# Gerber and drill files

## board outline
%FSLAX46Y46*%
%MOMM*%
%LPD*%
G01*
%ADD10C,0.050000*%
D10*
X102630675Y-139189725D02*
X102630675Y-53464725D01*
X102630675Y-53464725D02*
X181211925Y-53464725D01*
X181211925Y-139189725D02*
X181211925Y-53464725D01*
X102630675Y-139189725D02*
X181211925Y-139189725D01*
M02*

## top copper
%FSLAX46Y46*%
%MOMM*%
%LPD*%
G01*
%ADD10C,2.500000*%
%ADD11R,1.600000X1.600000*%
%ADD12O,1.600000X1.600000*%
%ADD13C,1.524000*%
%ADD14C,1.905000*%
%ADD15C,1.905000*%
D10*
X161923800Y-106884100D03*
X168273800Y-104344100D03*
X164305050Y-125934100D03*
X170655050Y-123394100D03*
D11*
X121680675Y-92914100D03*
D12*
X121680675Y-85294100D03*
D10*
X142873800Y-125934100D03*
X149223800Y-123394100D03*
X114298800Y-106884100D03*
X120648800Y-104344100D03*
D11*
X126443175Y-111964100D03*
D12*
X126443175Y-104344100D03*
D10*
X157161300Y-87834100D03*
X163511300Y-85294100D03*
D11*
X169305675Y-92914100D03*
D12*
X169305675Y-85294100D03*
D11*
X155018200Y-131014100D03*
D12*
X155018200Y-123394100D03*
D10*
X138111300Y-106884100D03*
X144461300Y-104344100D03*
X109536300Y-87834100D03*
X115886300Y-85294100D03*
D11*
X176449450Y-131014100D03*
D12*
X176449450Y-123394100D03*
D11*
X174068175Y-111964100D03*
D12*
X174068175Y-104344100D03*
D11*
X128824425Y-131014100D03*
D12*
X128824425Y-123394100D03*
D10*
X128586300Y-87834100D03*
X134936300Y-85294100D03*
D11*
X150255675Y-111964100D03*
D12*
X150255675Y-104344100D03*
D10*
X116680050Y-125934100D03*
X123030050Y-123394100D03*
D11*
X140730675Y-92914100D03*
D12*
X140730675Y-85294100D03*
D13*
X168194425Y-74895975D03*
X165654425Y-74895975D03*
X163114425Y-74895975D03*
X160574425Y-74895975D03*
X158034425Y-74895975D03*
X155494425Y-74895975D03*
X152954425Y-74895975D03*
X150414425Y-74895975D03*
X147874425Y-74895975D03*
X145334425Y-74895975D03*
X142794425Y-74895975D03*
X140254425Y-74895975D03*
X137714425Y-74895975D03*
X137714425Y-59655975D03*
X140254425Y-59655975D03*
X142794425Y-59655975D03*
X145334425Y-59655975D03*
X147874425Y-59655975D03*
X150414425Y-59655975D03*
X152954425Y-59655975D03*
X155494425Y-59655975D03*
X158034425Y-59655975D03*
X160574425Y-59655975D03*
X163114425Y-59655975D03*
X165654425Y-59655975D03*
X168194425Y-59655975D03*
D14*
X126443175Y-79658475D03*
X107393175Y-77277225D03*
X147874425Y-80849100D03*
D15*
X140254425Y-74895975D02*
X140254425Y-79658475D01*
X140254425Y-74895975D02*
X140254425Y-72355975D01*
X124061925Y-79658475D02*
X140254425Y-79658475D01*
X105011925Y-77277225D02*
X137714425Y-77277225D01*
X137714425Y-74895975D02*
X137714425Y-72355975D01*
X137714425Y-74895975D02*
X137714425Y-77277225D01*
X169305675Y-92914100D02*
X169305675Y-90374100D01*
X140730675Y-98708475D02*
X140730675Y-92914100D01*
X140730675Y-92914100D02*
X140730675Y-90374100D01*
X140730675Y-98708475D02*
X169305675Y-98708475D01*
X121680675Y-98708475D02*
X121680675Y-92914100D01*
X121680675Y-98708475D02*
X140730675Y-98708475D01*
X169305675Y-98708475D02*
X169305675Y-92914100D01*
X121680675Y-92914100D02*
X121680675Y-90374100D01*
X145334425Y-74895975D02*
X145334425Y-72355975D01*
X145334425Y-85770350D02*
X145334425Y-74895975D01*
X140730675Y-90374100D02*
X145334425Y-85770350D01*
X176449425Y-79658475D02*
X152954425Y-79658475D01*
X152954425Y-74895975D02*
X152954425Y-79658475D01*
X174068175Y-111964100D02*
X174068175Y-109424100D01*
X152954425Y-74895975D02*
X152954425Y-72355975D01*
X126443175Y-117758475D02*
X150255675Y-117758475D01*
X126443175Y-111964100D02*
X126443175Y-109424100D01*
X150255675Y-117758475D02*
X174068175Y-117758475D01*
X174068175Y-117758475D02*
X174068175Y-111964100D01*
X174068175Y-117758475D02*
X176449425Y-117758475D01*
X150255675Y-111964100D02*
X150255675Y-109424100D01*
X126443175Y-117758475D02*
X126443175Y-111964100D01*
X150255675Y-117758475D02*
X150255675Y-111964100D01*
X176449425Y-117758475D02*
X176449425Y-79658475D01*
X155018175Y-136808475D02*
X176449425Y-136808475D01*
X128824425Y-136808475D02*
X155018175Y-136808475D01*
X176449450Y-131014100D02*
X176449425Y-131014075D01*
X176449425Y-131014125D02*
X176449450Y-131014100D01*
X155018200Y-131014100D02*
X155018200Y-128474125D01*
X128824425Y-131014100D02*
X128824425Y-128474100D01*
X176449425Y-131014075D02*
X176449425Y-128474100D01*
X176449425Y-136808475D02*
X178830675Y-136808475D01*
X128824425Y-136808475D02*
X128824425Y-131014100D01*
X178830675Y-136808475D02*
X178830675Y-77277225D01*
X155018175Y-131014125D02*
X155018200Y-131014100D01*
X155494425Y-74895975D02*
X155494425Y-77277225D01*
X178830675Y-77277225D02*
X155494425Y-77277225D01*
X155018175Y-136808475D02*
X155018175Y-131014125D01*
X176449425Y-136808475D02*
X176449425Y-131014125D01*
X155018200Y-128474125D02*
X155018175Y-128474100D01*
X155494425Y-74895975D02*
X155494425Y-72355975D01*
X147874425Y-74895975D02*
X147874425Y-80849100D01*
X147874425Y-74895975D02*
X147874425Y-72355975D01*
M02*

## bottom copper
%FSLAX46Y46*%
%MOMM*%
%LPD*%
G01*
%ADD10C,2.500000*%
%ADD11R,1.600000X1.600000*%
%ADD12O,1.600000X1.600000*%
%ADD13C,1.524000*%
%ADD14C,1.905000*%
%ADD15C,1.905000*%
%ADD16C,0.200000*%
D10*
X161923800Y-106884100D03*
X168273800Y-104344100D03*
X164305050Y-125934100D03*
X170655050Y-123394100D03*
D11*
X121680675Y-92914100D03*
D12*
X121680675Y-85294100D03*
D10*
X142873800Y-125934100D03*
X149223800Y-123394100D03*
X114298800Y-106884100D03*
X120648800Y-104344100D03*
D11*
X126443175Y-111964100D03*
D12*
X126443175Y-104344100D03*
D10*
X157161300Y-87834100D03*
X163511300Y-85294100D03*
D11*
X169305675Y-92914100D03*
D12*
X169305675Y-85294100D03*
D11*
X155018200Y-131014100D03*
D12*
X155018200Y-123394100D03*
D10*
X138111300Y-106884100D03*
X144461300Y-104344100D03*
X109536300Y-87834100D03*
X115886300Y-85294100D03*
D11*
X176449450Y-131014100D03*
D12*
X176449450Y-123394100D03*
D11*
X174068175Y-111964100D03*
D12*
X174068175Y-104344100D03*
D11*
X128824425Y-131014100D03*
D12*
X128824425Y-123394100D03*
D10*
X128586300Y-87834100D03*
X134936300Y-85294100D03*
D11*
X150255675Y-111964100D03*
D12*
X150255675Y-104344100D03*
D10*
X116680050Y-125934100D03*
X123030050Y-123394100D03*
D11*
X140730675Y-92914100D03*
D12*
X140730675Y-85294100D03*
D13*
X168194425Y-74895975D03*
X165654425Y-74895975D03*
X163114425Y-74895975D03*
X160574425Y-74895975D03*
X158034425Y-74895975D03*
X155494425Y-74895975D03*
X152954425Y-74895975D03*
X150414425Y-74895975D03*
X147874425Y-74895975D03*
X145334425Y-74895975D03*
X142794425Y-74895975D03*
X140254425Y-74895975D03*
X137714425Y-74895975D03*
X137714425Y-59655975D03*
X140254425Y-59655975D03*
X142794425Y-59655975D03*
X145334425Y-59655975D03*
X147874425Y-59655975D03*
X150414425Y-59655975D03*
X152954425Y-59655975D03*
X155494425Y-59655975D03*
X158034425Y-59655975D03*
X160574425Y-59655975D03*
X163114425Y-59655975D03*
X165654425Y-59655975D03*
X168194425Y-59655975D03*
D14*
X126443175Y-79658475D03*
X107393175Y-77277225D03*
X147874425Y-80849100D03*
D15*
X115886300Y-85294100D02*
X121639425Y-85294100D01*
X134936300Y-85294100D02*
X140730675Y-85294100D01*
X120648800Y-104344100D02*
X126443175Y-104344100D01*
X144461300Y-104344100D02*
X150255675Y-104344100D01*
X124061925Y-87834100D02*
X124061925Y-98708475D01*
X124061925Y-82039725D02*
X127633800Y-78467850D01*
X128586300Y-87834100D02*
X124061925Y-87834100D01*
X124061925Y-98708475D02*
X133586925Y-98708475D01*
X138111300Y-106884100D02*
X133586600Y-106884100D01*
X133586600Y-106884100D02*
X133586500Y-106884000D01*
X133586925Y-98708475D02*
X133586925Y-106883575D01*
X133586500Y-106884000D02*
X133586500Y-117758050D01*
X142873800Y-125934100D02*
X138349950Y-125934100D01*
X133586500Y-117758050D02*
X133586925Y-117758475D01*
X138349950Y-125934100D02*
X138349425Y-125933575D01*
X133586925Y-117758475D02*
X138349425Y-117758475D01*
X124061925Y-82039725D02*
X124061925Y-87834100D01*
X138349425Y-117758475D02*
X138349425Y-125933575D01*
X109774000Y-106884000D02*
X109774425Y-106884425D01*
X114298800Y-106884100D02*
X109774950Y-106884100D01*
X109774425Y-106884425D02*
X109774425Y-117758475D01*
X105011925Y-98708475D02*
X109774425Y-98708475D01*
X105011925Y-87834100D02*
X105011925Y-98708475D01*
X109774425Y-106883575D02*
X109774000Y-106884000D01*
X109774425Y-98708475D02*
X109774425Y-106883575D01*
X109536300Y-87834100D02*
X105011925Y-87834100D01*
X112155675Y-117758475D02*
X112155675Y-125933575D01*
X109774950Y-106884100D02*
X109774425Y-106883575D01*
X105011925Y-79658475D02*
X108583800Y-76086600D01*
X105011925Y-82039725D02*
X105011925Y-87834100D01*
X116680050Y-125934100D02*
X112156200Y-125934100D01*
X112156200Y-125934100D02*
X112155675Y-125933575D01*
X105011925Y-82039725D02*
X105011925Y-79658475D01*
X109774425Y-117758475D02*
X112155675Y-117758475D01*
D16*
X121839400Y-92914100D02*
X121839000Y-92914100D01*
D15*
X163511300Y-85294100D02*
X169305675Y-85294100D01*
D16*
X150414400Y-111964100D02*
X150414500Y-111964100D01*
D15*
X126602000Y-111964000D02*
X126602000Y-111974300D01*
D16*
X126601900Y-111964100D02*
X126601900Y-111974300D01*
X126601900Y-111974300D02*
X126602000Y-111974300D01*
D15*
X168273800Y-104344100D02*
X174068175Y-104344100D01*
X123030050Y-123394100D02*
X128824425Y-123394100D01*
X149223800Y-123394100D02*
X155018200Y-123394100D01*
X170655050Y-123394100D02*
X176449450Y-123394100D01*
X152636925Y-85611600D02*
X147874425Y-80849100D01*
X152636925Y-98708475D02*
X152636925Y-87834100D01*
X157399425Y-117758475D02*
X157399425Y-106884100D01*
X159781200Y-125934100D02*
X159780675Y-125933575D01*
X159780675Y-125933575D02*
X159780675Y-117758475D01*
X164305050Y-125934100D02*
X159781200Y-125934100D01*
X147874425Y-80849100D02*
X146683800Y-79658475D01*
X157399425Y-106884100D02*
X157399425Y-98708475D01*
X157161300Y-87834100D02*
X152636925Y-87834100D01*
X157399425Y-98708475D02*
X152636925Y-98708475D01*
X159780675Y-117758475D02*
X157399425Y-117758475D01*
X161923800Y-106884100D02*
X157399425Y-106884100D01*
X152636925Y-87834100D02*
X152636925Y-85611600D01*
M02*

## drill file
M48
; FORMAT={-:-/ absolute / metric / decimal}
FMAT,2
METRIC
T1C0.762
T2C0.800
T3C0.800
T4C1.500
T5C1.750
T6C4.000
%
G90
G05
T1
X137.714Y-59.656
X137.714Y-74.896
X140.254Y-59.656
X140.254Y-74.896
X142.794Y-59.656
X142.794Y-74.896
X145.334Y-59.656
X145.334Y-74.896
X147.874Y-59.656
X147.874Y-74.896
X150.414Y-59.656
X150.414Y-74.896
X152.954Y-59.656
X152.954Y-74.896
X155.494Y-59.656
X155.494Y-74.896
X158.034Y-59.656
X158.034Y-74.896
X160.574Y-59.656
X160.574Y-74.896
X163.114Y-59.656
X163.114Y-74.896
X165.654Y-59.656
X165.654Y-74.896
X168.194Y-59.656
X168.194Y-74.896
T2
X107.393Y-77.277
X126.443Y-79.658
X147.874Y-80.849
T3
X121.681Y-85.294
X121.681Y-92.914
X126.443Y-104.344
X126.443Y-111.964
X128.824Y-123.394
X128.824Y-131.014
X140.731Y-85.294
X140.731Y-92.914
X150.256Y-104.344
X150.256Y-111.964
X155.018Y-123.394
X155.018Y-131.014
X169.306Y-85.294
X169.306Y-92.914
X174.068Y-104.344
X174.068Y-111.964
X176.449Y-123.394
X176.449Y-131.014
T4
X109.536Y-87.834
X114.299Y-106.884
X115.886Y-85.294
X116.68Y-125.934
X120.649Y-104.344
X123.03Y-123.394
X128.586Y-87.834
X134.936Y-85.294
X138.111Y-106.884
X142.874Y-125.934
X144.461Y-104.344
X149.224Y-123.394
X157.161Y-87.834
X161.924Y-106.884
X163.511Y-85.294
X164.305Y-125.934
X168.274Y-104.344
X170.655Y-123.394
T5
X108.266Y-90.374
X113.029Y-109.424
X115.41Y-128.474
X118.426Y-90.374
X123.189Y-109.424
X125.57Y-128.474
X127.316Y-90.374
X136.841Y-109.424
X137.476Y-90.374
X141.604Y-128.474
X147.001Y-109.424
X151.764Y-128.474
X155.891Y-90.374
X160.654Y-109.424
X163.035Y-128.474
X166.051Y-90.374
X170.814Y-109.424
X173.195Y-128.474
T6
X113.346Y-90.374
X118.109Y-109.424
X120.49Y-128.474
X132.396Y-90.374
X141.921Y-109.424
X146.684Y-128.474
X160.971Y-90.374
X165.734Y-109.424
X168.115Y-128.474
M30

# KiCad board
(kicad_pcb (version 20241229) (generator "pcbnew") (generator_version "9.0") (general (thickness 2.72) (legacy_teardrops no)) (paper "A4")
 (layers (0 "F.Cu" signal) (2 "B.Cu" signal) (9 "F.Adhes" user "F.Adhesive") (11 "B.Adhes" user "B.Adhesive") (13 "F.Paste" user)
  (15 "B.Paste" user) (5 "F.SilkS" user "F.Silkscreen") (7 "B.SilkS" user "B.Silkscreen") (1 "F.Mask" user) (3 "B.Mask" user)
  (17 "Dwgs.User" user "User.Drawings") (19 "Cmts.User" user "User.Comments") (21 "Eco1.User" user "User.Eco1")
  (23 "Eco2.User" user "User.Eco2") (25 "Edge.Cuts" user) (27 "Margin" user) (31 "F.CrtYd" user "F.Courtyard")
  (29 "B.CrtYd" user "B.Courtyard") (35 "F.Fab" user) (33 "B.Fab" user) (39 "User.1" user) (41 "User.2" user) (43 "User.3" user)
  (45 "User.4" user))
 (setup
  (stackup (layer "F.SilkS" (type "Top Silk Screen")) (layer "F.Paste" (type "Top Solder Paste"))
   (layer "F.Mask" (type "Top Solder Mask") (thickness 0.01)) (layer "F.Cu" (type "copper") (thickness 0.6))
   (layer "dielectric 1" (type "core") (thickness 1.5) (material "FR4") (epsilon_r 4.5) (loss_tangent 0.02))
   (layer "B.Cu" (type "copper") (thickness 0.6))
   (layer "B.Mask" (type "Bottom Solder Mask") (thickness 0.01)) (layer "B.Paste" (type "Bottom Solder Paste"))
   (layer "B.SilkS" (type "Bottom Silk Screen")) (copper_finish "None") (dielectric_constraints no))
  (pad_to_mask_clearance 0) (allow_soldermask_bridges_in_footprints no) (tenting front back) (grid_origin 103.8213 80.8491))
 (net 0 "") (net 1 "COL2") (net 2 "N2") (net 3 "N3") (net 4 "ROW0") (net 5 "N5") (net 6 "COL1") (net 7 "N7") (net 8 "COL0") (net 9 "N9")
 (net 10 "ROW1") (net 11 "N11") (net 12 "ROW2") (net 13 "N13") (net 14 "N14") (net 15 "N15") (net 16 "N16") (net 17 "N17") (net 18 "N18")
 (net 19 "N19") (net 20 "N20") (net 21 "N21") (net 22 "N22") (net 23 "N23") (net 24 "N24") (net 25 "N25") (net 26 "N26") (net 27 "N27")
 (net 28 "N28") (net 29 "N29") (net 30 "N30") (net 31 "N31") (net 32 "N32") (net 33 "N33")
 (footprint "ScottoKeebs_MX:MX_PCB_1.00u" (layer "F.Cu") (at 165.7338 109.4241)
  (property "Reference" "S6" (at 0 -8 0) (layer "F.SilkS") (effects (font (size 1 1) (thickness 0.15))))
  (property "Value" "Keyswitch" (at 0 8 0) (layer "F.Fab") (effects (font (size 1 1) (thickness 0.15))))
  (pad "" np_thru_hole circle (at -5.08 0) (size 1.75 1.75) (drill 1.75) (layers "*.Cu" "*.Mask"))
  (pad "" np_thru_hole circle (at 0 0) (size 4 4) (drill 4) (layers "*.Cu" "*.Mask"))
  (pad "" np_thru_hole circle (at 5.08 0) (size 1.75 1.75) (drill 1.75) (layers "*.Cu" "*.Mask"))
  (pad "1" thru_hole circle (at -3.81 -2.54) (size 2.5 2.5) (drill 1.5) (layers "*.Cu" "*.Mask") (remove_unused_layers no) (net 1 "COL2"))
  (pad "2" thru_hole circle (at 2.54 -5.08) (size 2.5 2.5) (drill 1.5) (layers "*.Cu" "*.Mask") (remove_unused_layers no) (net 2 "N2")))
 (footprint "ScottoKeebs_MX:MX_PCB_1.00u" (layer "F.Cu") (at 168.11505 128.4741)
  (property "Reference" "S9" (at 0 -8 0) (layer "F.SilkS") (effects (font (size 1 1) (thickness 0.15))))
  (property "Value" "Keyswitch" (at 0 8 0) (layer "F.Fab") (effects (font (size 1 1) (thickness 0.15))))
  (pad "" np_thru_hole circle (at -5.08 0) (size 1.75 1.75) (drill 1.75) (layers "*.Cu" "*.Mask"))
  (pad "" np_thru_hole circle (at 0 0) (size 4 4) (drill 4) (layers "*.Cu" "*.Mask"))
  (pad "" np_thru_hole circle (at 5.08 0) (size 1.75 1.75) (drill 1.75) (layers "*.Cu" "*.Mask"))
  (pad "1" thru_hole circle (at -3.81 -2.54) (size 2.5 2.5) (drill 1.5) (layers "*.Cu" "*.Mask") (remove_unused_layers no) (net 1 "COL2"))
  (pad "2" thru_hole circle (at 2.54 -5.08) (size 2.5 2.5) (drill 1.5) (layers "*.Cu" "*.Mask") (remove_unused_layers no) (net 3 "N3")))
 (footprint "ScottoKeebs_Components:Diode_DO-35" (layer "F.Cu") (at 121.680675 92.9141 90)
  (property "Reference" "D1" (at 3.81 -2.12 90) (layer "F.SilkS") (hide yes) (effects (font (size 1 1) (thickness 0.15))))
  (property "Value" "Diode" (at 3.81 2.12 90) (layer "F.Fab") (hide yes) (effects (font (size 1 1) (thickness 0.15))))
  (pad "1" thru_hole rect (at 0 0 90) (size 1.6 1.6) (drill 0.8) (layers "*.Cu" "*.Mask") (remove_unused_layers no) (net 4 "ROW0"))
  (pad "2" thru_hole oval (at 7.62 0 90) (size 1.6 1.6) (drill 0.8) (layers "*.Cu" "*.Mask") (remove_unused_layers no) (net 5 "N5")))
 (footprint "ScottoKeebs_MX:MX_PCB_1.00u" (layer "F.Cu") (at 146.6838 128.4741)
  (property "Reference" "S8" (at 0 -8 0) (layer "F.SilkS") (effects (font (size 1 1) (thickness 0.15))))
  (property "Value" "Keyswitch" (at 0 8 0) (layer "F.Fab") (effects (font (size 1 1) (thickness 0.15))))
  (pad "" np_thru_hole circle (at -5.08 0) (size 1.75 1.75) (drill 1.75) (layers "*.Cu" "*.Mask"))
  (pad "" np_thru_hole circle (at 0 0) (size 4 4) (drill 4) (layers "*.Cu" "*.Mask"))
  (pad "" np_thru_hole circle (at 5.08 0) (size 1.75 1.75) (drill 1.75) (layers "*.Cu" "*.Mask"))
  (pad "1" thru_hole circle (at -3.81 -2.54) (size 2.5 2.5) (drill 1.5) (layers "*.Cu" "*.Mask") (remove_unused_layers no) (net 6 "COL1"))
  (pad "2" thru_hole circle (at 2.54 -5.08) (size 2.5 2.5) (drill 1.5) (layers "*.Cu" "*.Mask") (remove_unused_layers no) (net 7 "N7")))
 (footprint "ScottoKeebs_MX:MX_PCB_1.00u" (layer "F.Cu") (at 118.1088 109.4241)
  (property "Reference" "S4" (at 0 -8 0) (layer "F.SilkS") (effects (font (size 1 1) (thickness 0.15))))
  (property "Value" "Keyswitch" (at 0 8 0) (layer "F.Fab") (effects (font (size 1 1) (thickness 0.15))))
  (pad "" np_thru_hole circle (at -5.08 0) (size 1.75 1.75) (drill 1.75) (layers "*.Cu" "*.Mask"))
  (pad "" np_thru_hole circle (at 0 0) (size 4 4) (drill 4) (layers "*.Cu" "*.Mask"))
  (pad "" np_thru_hole circle (at 5.08 0) (size 1.75 1.75) (drill 1.75) (layers "*.Cu" "*.Mask"))
  (pad "1" thru_hole circle (at -3.81 -2.54) (size 2.5 2.5) (drill 1.5) (layers "*.Cu" "*.Mask") (remove_unused_layers no) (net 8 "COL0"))
  (pad "2" thru_hole circle (at 2.54 -5.08) (size 2.5 2.5) (drill 1.5) (layers "*.Cu" "*.Mask") (remove_unused_layers no) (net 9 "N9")))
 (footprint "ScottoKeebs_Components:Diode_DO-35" (layer "F.Cu") (at 126.443175 111.9641 90)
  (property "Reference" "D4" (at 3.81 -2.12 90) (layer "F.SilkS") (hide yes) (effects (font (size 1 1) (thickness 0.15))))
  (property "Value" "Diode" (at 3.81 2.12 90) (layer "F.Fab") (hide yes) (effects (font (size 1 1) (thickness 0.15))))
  (pad "1" thru_hole rect (at 0 0 90) (size 1.6 1.6) (drill 0.8) (layers "*.Cu" "*.Mask") (remove_unused_layers no) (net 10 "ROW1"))
  (pad "2" thru_hole oval (at 7.62 0 90) (size 1.6 1.6) (drill 0.8) (layers "*.Cu" "*.Mask") (remove_unused_layers no) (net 9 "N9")))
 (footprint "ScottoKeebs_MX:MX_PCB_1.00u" (layer "F.Cu") (at 160.9713 90.3741)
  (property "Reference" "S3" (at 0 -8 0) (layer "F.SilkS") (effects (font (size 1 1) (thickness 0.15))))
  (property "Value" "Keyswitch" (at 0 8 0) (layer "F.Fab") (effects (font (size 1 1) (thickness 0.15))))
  (pad "" np_thru_hole circle (at -5.08 0) (size 1.75 1.75) (drill 1.75) (layers "*.Cu" "*.Mask"))
  (pad "" np_thru_hole circle (at 0 0) (size 4 4) (drill 4) (layers "*.Cu" "*.Mask"))
  (pad "" np_thru_hole circle (at 5.08 0) (size 1.75 1.75) (drill 1.75) (layers "*.Cu" "*.Mask"))
  (pad "1" thru_hole circle (at -3.81 -2.54) (size 2.5 2.5) (drill 1.5) (layers "*.Cu" "*.Mask") (remove_unused_layers no) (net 1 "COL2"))
  (pad "2" thru_hole circle (at 2.54 -5.08) (size 2.5 2.5) (drill 1.5) (layers "*.Cu" "*.Mask") (remove_unused_layers no) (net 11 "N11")))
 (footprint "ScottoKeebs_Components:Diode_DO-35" (layer "F.Cu") (at 169.305675 92.9141 90)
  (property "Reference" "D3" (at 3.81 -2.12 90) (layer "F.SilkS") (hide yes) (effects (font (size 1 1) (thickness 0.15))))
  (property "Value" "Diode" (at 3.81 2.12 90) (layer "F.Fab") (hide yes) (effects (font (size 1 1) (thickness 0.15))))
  (pad "1" thru_hole rect (at 0 0 90) (size 1.6 1.6) (drill 0.8) (layers "*.Cu" "*.Mask") (remove_unused_layers no) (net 4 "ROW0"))
  (pad "2" thru_hole oval (at 7.62 0 90) (size 1.6 1.6) (drill 0.8) (layers "*.Cu" "*.Mask") (remove_unused_layers no) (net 11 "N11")))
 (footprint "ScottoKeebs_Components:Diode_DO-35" (layer "F.Cu") (at 155.0182 131.0141 90)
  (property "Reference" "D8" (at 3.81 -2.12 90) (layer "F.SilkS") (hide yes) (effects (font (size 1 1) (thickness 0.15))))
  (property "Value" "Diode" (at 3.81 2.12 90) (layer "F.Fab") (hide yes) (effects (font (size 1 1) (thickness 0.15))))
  (pad "1" thru_hole rect (at 0 0 90) (size 1.6 1.6) (drill 0.8) (layers "*.Cu" "*.Mask") (remove_unused_layers no) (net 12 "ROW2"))
  (pad "2" thru_hole oval (at 7.62 0 90) (size 1.6 1.6) (drill 0.8) (layers "*.Cu" "*.Mask") (remove_unused_layers no) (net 7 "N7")))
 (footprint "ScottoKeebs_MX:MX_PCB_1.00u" (layer "F.Cu") (at 141.9213 109.4241)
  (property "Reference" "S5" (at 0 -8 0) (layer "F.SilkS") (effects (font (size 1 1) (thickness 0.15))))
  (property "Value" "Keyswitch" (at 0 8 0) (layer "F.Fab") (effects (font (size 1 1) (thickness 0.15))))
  (pad "" np_thru_hole circle (at -5.08 0) (size 1.75 1.75) (drill 1.75) (layers "*.Cu" "*.Mask"))
  (pad "" np_thru_hole circle (at 0 0) (size 4 4) (drill 4) (layers "*.Cu" "*.Mask"))
  (pad "" np_thru_hole circle (at 5.08 0) (size 1.75 1.75) (drill 1.75) (layers "*.Cu" "*.Mask"))
  (pad "1" thru_hole circle (at -3.81 -2.54) (size 2.5 2.5) (drill 1.5) (layers "*.Cu" "*.Mask") (remove_unused_layers no) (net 6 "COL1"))
  (pad "2" thru_hole circle (at 2.54 -5.08) (size 2.5 2.5) (drill 1.5) (layers "*.Cu" "*.Mask") (remove_unused_layers no) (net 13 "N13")))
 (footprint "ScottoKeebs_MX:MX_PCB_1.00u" (layer "F.Cu") (at 113.3463 90.3741)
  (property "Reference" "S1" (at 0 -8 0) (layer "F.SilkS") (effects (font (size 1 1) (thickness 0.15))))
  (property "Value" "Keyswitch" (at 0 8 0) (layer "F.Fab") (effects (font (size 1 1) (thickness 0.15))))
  (pad "" np_thru_hole circle (at -5.08 0) (size 1.75 1.75) (drill 1.75) (layers "*.Cu" "*.Mask"))
  (pad "" np_thru_hole circle (at 0 0) (size 4 4) (drill 4) (layers "*.Cu" "*.Mask"))
  (pad "" np_thru_hole circle (at 5.08 0) (size 1.75 1.75) (drill 1.75) (layers "*.Cu" "*.Mask"))
  (pad "1" thru_hole circle (at -3.81 -2.54) (size 2.5 2.5) (drill 1.5) (layers "*.Cu" "*.Mask") (remove_unused_layers no) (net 8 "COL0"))
  (pad "2" thru_hole circle (at 2.54 -5.08) (size 2.5 2.5) (drill 1.5) (layers "*.Cu" "*.Mask") (remove_unused_layers no) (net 5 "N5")))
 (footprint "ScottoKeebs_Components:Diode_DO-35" (layer "F.Cu") (at 176.44945 131.0141 90)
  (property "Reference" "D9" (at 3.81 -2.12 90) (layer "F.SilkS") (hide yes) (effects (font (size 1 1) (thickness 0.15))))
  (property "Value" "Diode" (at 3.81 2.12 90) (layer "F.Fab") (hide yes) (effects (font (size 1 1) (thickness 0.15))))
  (pad "1" thru_hole rect (at 0 0 90) (size 1.6 1.6) (drill 0.8) (layers "*.Cu" "*.Mask") (remove_unused_layers no) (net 12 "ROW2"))
  (pad "2" thru_hole oval (at 7.62 0 90) (size 1.6 1.6) (drill 0.8) (layers "*.Cu" "*.Mask") (remove_unused_layers no) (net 3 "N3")))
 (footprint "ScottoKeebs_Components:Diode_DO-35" (layer "F.Cu") (at 174.068175 111.9641 90)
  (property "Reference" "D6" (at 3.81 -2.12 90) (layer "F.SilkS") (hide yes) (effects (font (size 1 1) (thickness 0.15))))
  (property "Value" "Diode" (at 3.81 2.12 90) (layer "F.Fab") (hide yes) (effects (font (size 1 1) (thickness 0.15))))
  (pad "1" thru_hole rect (at 0 0 90) (size 1.6 1.6) (drill 0.8) (layers "*.Cu" "*.Mask") (remove_unused_layers no) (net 10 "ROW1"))
  (pad "2" thru_hole oval (at 7.62 0 90) (size 1.6 1.6) (drill 0.8) (layers "*.Cu" "*.Mask") (remove_unused_layers no) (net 2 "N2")))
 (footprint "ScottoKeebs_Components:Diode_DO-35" (layer "F.Cu") (at 128.824425 131.0141 90)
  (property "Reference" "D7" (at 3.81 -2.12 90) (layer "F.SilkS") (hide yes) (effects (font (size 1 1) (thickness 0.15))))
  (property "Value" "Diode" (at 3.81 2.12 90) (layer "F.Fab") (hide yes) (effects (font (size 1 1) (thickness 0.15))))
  (pad "1" thru_hole rect (at 0 0 90) (size 1.6 1.6) (drill 0.8) (layers "*.Cu" "*.Mask") (remove_unused_layers no) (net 12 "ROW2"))
  (pad "2" thru_hole oval (at 7.62 0 90) (size 1.6 1.6) (drill 0.8) (layers "*.Cu" "*.Mask") (remove_unused_layers no) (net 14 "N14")))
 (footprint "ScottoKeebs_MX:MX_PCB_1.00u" (layer "F.Cu") (at 132.3963 90.3741)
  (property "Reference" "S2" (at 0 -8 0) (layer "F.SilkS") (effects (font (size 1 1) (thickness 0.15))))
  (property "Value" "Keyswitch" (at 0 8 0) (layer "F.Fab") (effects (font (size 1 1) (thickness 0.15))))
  (pad "" np_thru_hole circle (at -5.08 0) (size 1.75 1.75) (drill 1.75) (layers "*.Cu" "*.Mask"))
  (pad "" np_thru_hole circle (at 0 0) (size 4 4) (drill 4) (layers "*.Cu" "*.Mask"))
  (pad "" np_thru_hole circle (at 5.08 0) (size 1.75 1.75) (drill 1.75) (layers "*.Cu" "*.Mask"))
  (pad "1" thru_hole circle (at -3.81 -2.54) (size 2.5 2.5) (drill 1.5) (layers "*.Cu" "*.Mask") (remove_unused_layers no) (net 6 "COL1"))
  (pad "2" thru_hole circle (at 2.54 -5.08) (size 2.5 2.5) (drill 1.5) (layers "*.Cu" "*.Mask") (remove_unused_layers no) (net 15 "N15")))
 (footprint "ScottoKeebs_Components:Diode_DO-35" (layer "F.Cu") (at 150.255675 111.9641 90)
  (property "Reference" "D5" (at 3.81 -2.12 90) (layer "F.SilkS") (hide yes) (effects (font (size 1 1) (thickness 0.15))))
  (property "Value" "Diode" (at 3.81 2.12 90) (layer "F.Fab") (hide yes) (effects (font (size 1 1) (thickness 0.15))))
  (pad "1" thru_hole rect (at 0 0 90) (size 1.6 1.6) (drill 0.8) (layers "*.Cu" "*.Mask") (remove_unused_layers no) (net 10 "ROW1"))
  (pad "2" thru_hole oval (at 7.62 0 90) (size 1.6 1.6) (drill 0.8) (layers "*.Cu" "*.Mask") (remove_unused_layers no) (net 13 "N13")))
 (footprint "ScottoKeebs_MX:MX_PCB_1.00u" (layer "F.Cu") (at 120.49005 128.4741)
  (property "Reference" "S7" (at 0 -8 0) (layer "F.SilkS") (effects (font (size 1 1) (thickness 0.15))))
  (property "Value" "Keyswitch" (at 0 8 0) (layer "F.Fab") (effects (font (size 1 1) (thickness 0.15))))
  (pad "" np_thru_hole circle (at -5.08 0) (size 1.75 1.75) (drill 1.75) (layers "*.Cu" "*.Mask"))
  (pad "" np_thru_hole circle (at 0 0) (size 4 4) (drill 4) (layers "*.Cu" "*.Mask"))
  (pad "" np_thru_hole circle (at 5.08 0) (size 1.75 1.75) (drill 1.75) (layers "*.Cu" "*.Mask"))
  (pad "1" thru_hole circle (at -3.81 -2.54) (size 2.5 2.5) (drill 1.5) (layers "*.Cu" "*.Mask") (remove_unused_layers no) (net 8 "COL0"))
  (pad "2" thru_hole circle (at 2.54 -5.08) (size 2.5 2.5) (drill 1.5) (layers "*.Cu" "*.Mask") (remove_unused_layers no) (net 14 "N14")))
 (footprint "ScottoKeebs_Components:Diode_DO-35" (layer "F.Cu") (at 140.730675 92.9141 90)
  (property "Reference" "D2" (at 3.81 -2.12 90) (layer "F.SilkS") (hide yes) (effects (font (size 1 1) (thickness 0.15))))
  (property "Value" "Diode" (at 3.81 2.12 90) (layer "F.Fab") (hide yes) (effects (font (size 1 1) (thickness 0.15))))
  (pad "1" thru_hole rect (at 0 0 90) (size 1.6 1.6) (drill 0.8) (layers "*.Cu" "*.Mask") (remove_unused_layers no) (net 4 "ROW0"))
  (pad "2" thru_hole oval (at 7.62 0 90) (size 1.6 1.6) (drill 0.8) (layers "*.Cu" "*.Mask") (remove_unused_layers no) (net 15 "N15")))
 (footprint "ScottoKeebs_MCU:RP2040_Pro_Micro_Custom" (layer "B.Cu") (at 151.684425 67.275975 90)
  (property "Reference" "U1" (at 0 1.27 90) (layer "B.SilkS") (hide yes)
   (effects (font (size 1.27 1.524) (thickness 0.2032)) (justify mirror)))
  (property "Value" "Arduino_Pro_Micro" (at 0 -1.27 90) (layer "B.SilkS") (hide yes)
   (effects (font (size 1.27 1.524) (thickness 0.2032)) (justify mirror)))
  (pad "1" thru_hole circle (at -7.62 16.51 90) (size 1.524 1.524) (drill 0.762) (layers "*.Cu" "*.Mask") (remove_unused_layers no))
  (pad "2" thru_hole circle (at -7.62 13.97 90) (size 1.524 1.524) (drill 0.762) (layers "*.Cu" "*.Mask") (remove_unused_layers no)
   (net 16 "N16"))
  (pad "3" thru_hole circle (at -7.62 11.43 90) (size 1.524 1.524) (drill 0.762) (layers "*.Cu" "*.Mask") (remove_unused_layers no)
   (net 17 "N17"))
  (pad "4" thru_hole circle (at -7.62 8.89 90) (size 1.524 1.524) (drill 0.762) (layers "*.Cu" "*.Mask") (remove_unused_layers no)
   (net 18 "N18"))
  (pad "5" thru_hole circle (at -7.62 6.35 90) (size 1.524 1.524) (drill 0.762) (layers "*.Cu" "*.Mask") (remove_unused_layers no)
   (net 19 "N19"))
  (pad "6" thru_hole circle (at -7.62 3.81 90) (size 1.524 1.524) (drill 0.762) (layers "*.Cu" "*.Mask") (remove_unused_layers no)
   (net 12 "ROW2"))
  (pad "7" thru_hole circle (at -7.62 1.27 90) (size 1.524 1.524) (drill 0.762) (layers "*.Cu" "*.Mask") (remove_unused_layers no)
   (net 10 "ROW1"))
  (pad "8" thru_hole circle (at -7.62 -1.27 90) (size 1.524 1.524) (drill 0.762) (layers "*.Cu" "*.Mask") (remove_unused_layers no)
   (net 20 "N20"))
  (pad "9" thru_hole circle (at -7.62 -3.81 90) (size 1.524 1.524) (drill 0.762) (layers "*.Cu" "*.Mask") (remove_unused_layers no)
   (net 1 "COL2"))
  (pad "10" thru_hole circle (at -7.62 -6.35 90) (size 1.524 1.524) (drill 0.762) (layers "*.Cu" "*.Mask") (remove_unused_layers no)
   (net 4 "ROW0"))
  (pad "11" thru_hole circle (at -7.62 -8.89 90) (size 1.524 1.524) (drill 0.762) (layers "*.Cu" "*.Mask") (remove_unused_layers no)
   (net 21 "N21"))
  (pad "12" thru_hole circle (at -7.62 -11.43 90) (size 1.524 1.524) (drill 0.762) (layers "*.Cu" "*.Mask") (remove_unused_layers no)
   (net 6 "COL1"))
  (pad "13" thru_hole circle (at -7.62 -13.97 90) (size 1.524 1.524) (drill 0.762) (layers "*.Cu" "*.Mask") (remove_unused_layers no)
   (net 8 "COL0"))
  (pad "19" thru_hole circle (at 7.62 -13.97 90) (size 1.524 1.524) (drill 0.762) (layers "*.Cu" "*.Mask") (remove_unused_layers no)
   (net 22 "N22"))
  (pad "20" thru_hole circle (at 7.62 -11.43 90) (size 1.524 1.524) (drill 0.762) (layers "*.Cu" "*.Mask") (remove_unused_layers no)
   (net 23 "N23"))
  (pad "21" thru_hole circle (at 7.62 -8.89 90) (size 1.524 1.524) (drill 0.762) (layers "*.Cu" "*.Mask") (remove_unused_layers no)
   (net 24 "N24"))
  (pad "22" thru_hole circle (at 7.62 -6.35 90) (size 1.524 1.524) (drill 0.762) (layers "*.Cu" "*.Mask") (remove_unused_layers no)
   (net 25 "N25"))
  (pad "23" thru_hole circle (at 7.62 -3.81 90) (size 1.524 1.524) (drill 0.762) (layers "*.Cu" "*.Mask") (remove_unused_layers no)
   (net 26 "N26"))
  (pad "24" thru_hole circle (at 7.62 -1.27 90) (size 1.524 1.524) (drill 0.762) (layers "*.Cu" "*.Mask") (remove_unused_layers no)
   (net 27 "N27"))
  (pad "25" thru_hole circle (at 7.62 1.27 90) (size 1.524 1.524) (drill 0.762) (layers "*.Cu" "*.Mask") (remove_unused_layers no)
   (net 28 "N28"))
  (pad "26" thru_hole circle (at 7.62 3.81 90) (size 1.524 1.524) (drill 0.762) (layers "*.Cu" "*.Mask") (remove_unused_layers no)
   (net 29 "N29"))
  (pad "27" thru_hole circle (at 7.62 6.35 90) (size 1.524 1.524) (drill 0.762) (layers "*.Cu" "*.Mask") (remove_unused_layers no)
   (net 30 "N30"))
  (pad "28" thru_hole circle (at 7.62 8.89 90) (size 1.524 1.524) (drill 0.762) (layers "*.Cu" "*.Mask") (remove_unused_layers no)
   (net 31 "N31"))
  (pad "29" thru_hole circle (at 7.62 11.43 90) (size 1.524 1.524) (drill 0.762) (layers "*.Cu" "*.Mask") (remove_unused_layers no)
   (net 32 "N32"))
  (pad "30" thru_hole circle (at 7.62 13.97 90) (size 1.524 1.524) (drill 0.762) (layers "*.Cu" "*.Mask") (remove_unused_layers no)
   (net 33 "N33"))
  (pad "31" thru_hole circle (at 7.62 16.51 90) (size 1.524 1.524) (drill 0.762) (layers "*.Cu" "*.Mask") (remove_unused_layers no)))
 (gr_line (start 102.630675 139.189725) (end 102.630675 53.464725) (stroke (width 0.05) (type default)) (layer "Edge.Cuts"))
 (gr_line (start 102.630675 53.464725) (end 181.211925 53.464725) (stroke (width 0.05) (type default)) (layer "Edge.Cuts"))
 (gr_line (start 181.211925 139.189725) (end 181.211925 53.464725) (stroke (width 0.05) (type default)) (layer "Edge.Cuts"))
 (gr_line (start 102.630675 139.189725) (end 181.211925 139.189725) (stroke (width 0.05) (type default)) (layer "Edge.Cuts"))
 (segment (start 115.8863 85.2941) (end 121.639425 85.2941) (width 1.905) (layer "B.Cu") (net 5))
 (segment (start 134.9363 85.2941) (end 140.730675 85.2941) (width 1.905) (layer "B.Cu") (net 15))
 (segment (start 120.6488 104.3441) (end 126.443175 104.3441) (width 1.905) (layer "B.Cu") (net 9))
 (segment (start 144.4613 104.3441) (end 150.255675 104.3441) (width 1.905) (layer "B.Cu") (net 13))
 (segment (start 140.254425 74.895975) (end 140.254425 79.658475) (width 1.905) (layer "F.Cu") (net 6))
 (segment (start 140.254425 74.895975) (end 140.254425 72.355975) (width 1.905) (layer "F.Cu") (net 6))
 (segment (start 124.061925 79.658475) (end 140.254425 79.658475) (width 1.905) (layer "F.Cu") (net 6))
 (via (at 126.443175 79.658475) (size 1.905) (drill 0.8) (layers "F.Cu" "B.Cu") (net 6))
 (segment (start 124.061925 87.8341) (end 124.061925 98.708475) (width 1.905) (layer "B.Cu") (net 6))
 (segment (start 124.061925 82.039725) (end 127.6338 78.46785) (width 1.905) (layer "B.Cu") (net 6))
 (segment (start 128.5863 87.8341) (end 124.061925 87.8341) (width 1.905) (layer "B.Cu") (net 6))
 (segment (start 124.061925 98.708475) (end 133.586925 98.708475) (width 1.905) (layer "B.Cu") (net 6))
 (segment (start 138.1113 106.8841) (end 133.5866 106.8841) (width 1.905) (layer "B.Cu") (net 6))
 (segment (start 133.5866 106.8841) (end 133.5865 106.884) (width 1.905) (layer "B.Cu") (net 6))
 (segment (start 133.586925 98.708475) (end 133.586925 106.883575) (width 1.905) (layer "B.Cu") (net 6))
 (segment (start 133.5865 106.884) (end 133.5865 117.75805) (width 1.905) (layer "B.Cu") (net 6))
 (segment (start 142.8738 125.9341) (end 138.34995 125.9341) (width 1.905) (layer "B.Cu") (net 6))
 (segment (start 133.5865 117.75805) (end 133.586925 117.758475) (width 1.905) (layer "B.Cu") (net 6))
 (segment (start 138.34995 125.9341) (end 138.349425 125.933575) (width 1.905) (layer "B.Cu") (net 6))
 (segment (start 133.586925 117.758475) (end 138.349425 117.758475) (width 1.905) (layer "B.Cu") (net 6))
 (segment (start 124.061925 82.039725) (end 124.061925 87.8341) (width 1.905) (layer "B.Cu") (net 6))
 (segment (start 138.349425 117.758475) (end 138.349425 125.933575) (width 1.905) (layer "B.Cu") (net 6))
 (segment (start 105.011925 77.277225) (end 137.714425 77.277225) (width 1.905) (layer "F.Cu") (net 8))
 (segment (start 137.714425 74.895975) (end 137.714425 72.355975) (width 1.905) (layer "F.Cu") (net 8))
 (segment (start 137.714425 74.895975) (end 137.714425 77.277225) (width 1.905) (layer "F.Cu") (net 8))
 (via (at 107.393175 77.277225) (size 1.905) (drill 0.8) (layers "F.Cu" "B.Cu") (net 8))
 (segment (start 109.774 106.884) (end 109.774425 106.884425) (width 1.905) (layer "B.Cu") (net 8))
 (segment (start 114.2988 106.8841) (end 109.77495 106.8841) (width 1.905) (layer "B.Cu") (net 8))
 (segment (start 109.774425 106.884425) (end 109.774425 117.758475) (width 1.905) (layer "B.Cu") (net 8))
 (segment (start 105.011925 98.708475) (end 109.774425 98.708475) (width 1.905) (layer "B.Cu") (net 8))
 (segment (start 105.011925 87.8341) (end 105.011925 98.708475) (width 1.905) (layer "B.Cu") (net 8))
 (segment (start 109.774425 106.883575) (end 109.774 106.884) (width 1.905) (layer "B.Cu") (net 8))
 (segment (start 109.774425 98.708475) (end 109.774425 106.883575) (width 1.905) (layer "B.Cu") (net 8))
 (segment (start 109.5363 87.8341) (end 105.011925 87.8341) (width 1.905) (layer "B.Cu") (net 8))
 (segment (start 112.155675 117.758475) (end 112.155675 125.933575) (width 1.905) (layer "B.Cu") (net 8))
 (segment (start 109.77495 106.8841) (end 109.774425 106.883575) (width 1.905) (layer "B.Cu") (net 8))
 (segment (start 105.011925 79.658475) (end 108.5838 76.0866) (width 1.905) (layer "B.Cu") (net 8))
 (segment (start 105.011925 82.039725) (end 105.011925 87.8341) (width 1.905) (layer "B.Cu") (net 8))
 (segment (start 116.68005 125.9341) (end 112.1562 125.9341) (width 1.905) (layer "B.Cu") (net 8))
 (segment (start 112.1562 125.9341) (end 112.155675 125.933575) (width 1.905) (layer "B.Cu") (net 8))
 (segment (start 105.011925 82.039725) (end 105.011925 79.658475) (width 1.905) (layer "B.Cu") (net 8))
 (segment (start 109.774425 117.758475) (end 112.155675 117.758475) (width 1.905) (layer "B.Cu") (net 8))
 (segment (start 169.305675 92.9141) (end 169.305675 90.3741) (width 1.905) (layer "F.Cu") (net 4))
 (segment (start 140.730675 98.708475) (end 140.730675 92.9141) (width 1.905) (layer "F.Cu") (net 4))
 (segment (start 140.730675 92.9141) (end 140.730675 90.3741) (width 1.905) (layer "F.Cu") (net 4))
 (segment (start 140.730675 98.708475) (end 169.305675 98.708475) (width 1.905) (layer "F.Cu") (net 4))
 (segment (start 121.680675 98.708475) (end 121.680675 92.9141) (width 1.905) (layer "F.Cu") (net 4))
 (segment (start 121.680675 98.708475) (end 140.730675 98.708475) (width 1.905) (layer "F.Cu") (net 4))
 (segment (start 169.305675 98.708475) (end 169.305675 92.9141) (width 1.905) (layer "F.Cu") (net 4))
 (segment (start 121.680675 92.9141) (end 121.680675 90.3741) (width 1.905) (layer "F.Cu") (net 4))
 (segment (start 145.334425 74.895975) (end 145.334425 72.355975) (width 1.905) (layer "F.Cu") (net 4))
 (segment (start 145.334425 85.77035) (end 145.334425 74.895975) (width 1.905) (layer "F.Cu") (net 4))
 (segment (start 140.730675 90.3741) (end 145.334425 85.77035) (width 1.905) (layer "F.Cu") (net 4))
 (segment (start 121.8394 92.9141) (end 121.839 92.9141) (width 0.2) (layer "B.Cu") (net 4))
 (segment (start 163.5113 85.2941) (end 169.305675 85.2941) (width 1.905) (layer "B.Cu") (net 11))
 (segment (start 176.449425 79.658475) (end 152.954425 79.658475) (width 1.905) (layer "F.Cu") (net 10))
 (segment (start 152.954425 74.895975) (end 152.954425 79.658475) (width 1.905) (layer "F.Cu") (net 10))
 (segment (start 174.068175 111.9641) (end 174.068175 109.4241) (width 1.905) (layer "F.Cu") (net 10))
 (segment (start 152.954425 74.895975) (end 152.954425 72.355975) (width 1.905) (layer "F.Cu") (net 10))
 (segment (start 126.443175 117.758475) (end 150.255675 117.758475) (width 1.905) (layer "F.Cu") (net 10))
 (segment (start 126.443175 111.9641) (end 126.443175 109.4241) (width 1.905) (layer "F.Cu") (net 10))
 (segment (start 150.255675 117.758475) (end 174.068175 117.758475) (width 1.905) (layer "F.Cu") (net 10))
 (segment (start 174.068175 117.758475) (end 174.068175 111.9641) (width 1.905) (layer "F.Cu") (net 10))
 (segment (start 174.068175 117.758475) (end 176.449425 117.758475) (width 1.905) (layer "F.Cu") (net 10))
 (segment (start 150.255675 111.9641) (end 150.255675 109.4241) (width 1.905) (layer "F.Cu") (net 10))
 (segment (start 126.443175 117.758475) (end 126.443175 111.9641) (width 1.905) (layer "F.Cu") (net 10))
 (segment (start 150.255675 117.758475) (end 150.255675 111.9641) (width 1.905) (layer "F.Cu") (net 10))
 (segment (start 176.449425 117.758475) (end 176.449425 79.658475) (width 1.905) (layer "F.Cu") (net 10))
 (segment (start 150.4144 111.9641) (end 150.4145 111.9641) (width 0.2) (layer "B.Cu") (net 10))
 (segment (start 126.602 111.964) (end 126.602 111.9743) (width 1.905) (layer "B.Cu") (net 10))
 (segment (start 126.6019 111.9641) (end 126.6019 111.9743) (width 0.2) (layer "B.Cu") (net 10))
 (segment (start 126.6019 111.9743) (end 126.602 111.9743) (width 0.2) (layer "B.Cu") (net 10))
 (segment (start 168.2738 104.3441) (end 174.068175 104.3441) (width 1.905) (layer "B.Cu") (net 2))
 (segment (start 155.018175 136.808475) (end 176.449425 136.808475) (width 1.905) (layer "F.Cu") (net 12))
 (segment (start 128.824425 136.808475) (end 155.018175 136.808475) (width 1.905) (layer "F.Cu") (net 12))
 (segment (start 176.44945 131.0141) (end 176.449425 131.014075) (width 1.905) (layer "F.Cu") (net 12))
 (segment (start 176.449425 131.014125) (end 176.44945 131.0141) (width 1.905) (layer "F.Cu") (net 12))
 (segment (start 155.0182 131.0141) (end 155.0182 128.474125) (width 1.905) (layer "F.Cu") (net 12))
 (segment (start 128.824425 131.0141) (end 128.824425 128.4741) (width 1.905) (layer "F.Cu") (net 12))
 (segment (start 176.449425 131.014075) (end 176.449425 128.4741) (width 1.905) (layer "F.Cu") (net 12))
 (segment (start 176.449425 136.808475) (end 178.830675 136.808475) (width 1.905) (layer "F.Cu") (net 12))
 (segment (start 128.824425 136.808475) (end 128.824425 131.0141) (width 1.905) (layer "F.Cu") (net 12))
 (segment (start 178.830675 136.808475) (end 178.830675 77.277225) (width 1.905) (layer "F.Cu") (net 12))
 (segment (start 155.018175 131.014125) (end 155.0182 131.0141) (width 1.905) (layer "F.Cu") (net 12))
 (segment (start 155.494425 74.895975) (end 155.494425 77.277225) (width 1.905) (layer "F.Cu") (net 12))
 (segment (start 178.830675 77.277225) (end 155.494425 77.277225) (width 1.905) (layer "F.Cu") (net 12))
 (segment (start 155.018175 136.808475) (end 155.018175 131.014125) (width 1.905) (layer "F.Cu") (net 12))
 (segment (start 176.449425 136.808475) (end 176.449425 131.014125) (width 1.905) (layer "F.Cu") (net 12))
 (segment (start 155.0182 128.474125) (end 155.018175 128.4741) (width 1.905) (layer "F.Cu") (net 12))
 (segment (start 155.494425 74.895975) (end 155.494425 72.355975) (width 1.905) (layer "F.Cu") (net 12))
 (segment (start 123.03005 123.3941) (end 128.824425 123.3941) (width 1.905) (layer "B.Cu") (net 14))
 (segment (start 149.2238 123.3941) (end 155.0182 123.3941) (width 1.905) (layer "B.Cu") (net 7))
 (segment (start 170.65505 123.3941) (end 176.44945 123.3941) (width 1.905) (layer "B.Cu") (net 3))
 (segment (start 147.874425 74.895975) (end 147.874425 80.8491) (width 1.905) (layer "F.Cu") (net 1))
 (segment (start 147.874425 74.895975) (end 147.874425 72.355975) (width 1.905) (layer "F.Cu") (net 1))
 (via (at 147.874425 80.8491) (size 1.905) (drill 0.8) (layers "F.Cu" "B.Cu") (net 1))
 (segment (start 152.636925 85.6116) (end 147.874425 80.8491) (width 1.905) (layer "B.Cu") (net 1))
 (segment (start 152.636925 98.708475) (end 152.636925 87.8341) (width 1.905) (layer "B.Cu") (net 1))
 (segment (start 157.399425 117.758475) (end 157.399425 106.8841) (width 1.905) (layer "B.Cu") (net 1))
 (segment (start 159.7812 125.9341) (end 159.780675 125.933575) (width 1.905) (layer "B.Cu") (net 1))
 (segment (start 159.780675 125.933575) (end 159.780675 117.758475) (width 1.905) (layer "B.Cu") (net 1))
 (segment (start 164.30505 125.9341) (end 159.7812 125.9341) (width 1.905) (layer "B.Cu") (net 1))
 (segment (start 147.874425 80.8491) (end 146.6838 79.658475) (width 1.905) (layer "B.Cu") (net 1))
 (segment (start 157.399425 106.8841) (end 157.399425 98.708475) (width 1.905) (layer "B.Cu") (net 1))
 (segment (start 157.1613 87.8341) (end 152.636925 87.8341) (width 1.905) (layer "B.Cu") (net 1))
 (segment (start 157.399425 98.708475) (end 152.636925 98.708475) (width 1.905) (layer "B.Cu") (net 1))
 (segment (start 159.780675 117.758475) (end 157.399425 117.758475) (width 1.905) (layer "B.Cu") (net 1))
 (segment (start 161.9238 106.8841) (end 157.399425 106.8841) (width 1.905) (layer "B.Cu") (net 1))
 (segment (start 152.636925 87.8341) (end 152.636925 85.6116) (width 1.905) (layer "B.Cu") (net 1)))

